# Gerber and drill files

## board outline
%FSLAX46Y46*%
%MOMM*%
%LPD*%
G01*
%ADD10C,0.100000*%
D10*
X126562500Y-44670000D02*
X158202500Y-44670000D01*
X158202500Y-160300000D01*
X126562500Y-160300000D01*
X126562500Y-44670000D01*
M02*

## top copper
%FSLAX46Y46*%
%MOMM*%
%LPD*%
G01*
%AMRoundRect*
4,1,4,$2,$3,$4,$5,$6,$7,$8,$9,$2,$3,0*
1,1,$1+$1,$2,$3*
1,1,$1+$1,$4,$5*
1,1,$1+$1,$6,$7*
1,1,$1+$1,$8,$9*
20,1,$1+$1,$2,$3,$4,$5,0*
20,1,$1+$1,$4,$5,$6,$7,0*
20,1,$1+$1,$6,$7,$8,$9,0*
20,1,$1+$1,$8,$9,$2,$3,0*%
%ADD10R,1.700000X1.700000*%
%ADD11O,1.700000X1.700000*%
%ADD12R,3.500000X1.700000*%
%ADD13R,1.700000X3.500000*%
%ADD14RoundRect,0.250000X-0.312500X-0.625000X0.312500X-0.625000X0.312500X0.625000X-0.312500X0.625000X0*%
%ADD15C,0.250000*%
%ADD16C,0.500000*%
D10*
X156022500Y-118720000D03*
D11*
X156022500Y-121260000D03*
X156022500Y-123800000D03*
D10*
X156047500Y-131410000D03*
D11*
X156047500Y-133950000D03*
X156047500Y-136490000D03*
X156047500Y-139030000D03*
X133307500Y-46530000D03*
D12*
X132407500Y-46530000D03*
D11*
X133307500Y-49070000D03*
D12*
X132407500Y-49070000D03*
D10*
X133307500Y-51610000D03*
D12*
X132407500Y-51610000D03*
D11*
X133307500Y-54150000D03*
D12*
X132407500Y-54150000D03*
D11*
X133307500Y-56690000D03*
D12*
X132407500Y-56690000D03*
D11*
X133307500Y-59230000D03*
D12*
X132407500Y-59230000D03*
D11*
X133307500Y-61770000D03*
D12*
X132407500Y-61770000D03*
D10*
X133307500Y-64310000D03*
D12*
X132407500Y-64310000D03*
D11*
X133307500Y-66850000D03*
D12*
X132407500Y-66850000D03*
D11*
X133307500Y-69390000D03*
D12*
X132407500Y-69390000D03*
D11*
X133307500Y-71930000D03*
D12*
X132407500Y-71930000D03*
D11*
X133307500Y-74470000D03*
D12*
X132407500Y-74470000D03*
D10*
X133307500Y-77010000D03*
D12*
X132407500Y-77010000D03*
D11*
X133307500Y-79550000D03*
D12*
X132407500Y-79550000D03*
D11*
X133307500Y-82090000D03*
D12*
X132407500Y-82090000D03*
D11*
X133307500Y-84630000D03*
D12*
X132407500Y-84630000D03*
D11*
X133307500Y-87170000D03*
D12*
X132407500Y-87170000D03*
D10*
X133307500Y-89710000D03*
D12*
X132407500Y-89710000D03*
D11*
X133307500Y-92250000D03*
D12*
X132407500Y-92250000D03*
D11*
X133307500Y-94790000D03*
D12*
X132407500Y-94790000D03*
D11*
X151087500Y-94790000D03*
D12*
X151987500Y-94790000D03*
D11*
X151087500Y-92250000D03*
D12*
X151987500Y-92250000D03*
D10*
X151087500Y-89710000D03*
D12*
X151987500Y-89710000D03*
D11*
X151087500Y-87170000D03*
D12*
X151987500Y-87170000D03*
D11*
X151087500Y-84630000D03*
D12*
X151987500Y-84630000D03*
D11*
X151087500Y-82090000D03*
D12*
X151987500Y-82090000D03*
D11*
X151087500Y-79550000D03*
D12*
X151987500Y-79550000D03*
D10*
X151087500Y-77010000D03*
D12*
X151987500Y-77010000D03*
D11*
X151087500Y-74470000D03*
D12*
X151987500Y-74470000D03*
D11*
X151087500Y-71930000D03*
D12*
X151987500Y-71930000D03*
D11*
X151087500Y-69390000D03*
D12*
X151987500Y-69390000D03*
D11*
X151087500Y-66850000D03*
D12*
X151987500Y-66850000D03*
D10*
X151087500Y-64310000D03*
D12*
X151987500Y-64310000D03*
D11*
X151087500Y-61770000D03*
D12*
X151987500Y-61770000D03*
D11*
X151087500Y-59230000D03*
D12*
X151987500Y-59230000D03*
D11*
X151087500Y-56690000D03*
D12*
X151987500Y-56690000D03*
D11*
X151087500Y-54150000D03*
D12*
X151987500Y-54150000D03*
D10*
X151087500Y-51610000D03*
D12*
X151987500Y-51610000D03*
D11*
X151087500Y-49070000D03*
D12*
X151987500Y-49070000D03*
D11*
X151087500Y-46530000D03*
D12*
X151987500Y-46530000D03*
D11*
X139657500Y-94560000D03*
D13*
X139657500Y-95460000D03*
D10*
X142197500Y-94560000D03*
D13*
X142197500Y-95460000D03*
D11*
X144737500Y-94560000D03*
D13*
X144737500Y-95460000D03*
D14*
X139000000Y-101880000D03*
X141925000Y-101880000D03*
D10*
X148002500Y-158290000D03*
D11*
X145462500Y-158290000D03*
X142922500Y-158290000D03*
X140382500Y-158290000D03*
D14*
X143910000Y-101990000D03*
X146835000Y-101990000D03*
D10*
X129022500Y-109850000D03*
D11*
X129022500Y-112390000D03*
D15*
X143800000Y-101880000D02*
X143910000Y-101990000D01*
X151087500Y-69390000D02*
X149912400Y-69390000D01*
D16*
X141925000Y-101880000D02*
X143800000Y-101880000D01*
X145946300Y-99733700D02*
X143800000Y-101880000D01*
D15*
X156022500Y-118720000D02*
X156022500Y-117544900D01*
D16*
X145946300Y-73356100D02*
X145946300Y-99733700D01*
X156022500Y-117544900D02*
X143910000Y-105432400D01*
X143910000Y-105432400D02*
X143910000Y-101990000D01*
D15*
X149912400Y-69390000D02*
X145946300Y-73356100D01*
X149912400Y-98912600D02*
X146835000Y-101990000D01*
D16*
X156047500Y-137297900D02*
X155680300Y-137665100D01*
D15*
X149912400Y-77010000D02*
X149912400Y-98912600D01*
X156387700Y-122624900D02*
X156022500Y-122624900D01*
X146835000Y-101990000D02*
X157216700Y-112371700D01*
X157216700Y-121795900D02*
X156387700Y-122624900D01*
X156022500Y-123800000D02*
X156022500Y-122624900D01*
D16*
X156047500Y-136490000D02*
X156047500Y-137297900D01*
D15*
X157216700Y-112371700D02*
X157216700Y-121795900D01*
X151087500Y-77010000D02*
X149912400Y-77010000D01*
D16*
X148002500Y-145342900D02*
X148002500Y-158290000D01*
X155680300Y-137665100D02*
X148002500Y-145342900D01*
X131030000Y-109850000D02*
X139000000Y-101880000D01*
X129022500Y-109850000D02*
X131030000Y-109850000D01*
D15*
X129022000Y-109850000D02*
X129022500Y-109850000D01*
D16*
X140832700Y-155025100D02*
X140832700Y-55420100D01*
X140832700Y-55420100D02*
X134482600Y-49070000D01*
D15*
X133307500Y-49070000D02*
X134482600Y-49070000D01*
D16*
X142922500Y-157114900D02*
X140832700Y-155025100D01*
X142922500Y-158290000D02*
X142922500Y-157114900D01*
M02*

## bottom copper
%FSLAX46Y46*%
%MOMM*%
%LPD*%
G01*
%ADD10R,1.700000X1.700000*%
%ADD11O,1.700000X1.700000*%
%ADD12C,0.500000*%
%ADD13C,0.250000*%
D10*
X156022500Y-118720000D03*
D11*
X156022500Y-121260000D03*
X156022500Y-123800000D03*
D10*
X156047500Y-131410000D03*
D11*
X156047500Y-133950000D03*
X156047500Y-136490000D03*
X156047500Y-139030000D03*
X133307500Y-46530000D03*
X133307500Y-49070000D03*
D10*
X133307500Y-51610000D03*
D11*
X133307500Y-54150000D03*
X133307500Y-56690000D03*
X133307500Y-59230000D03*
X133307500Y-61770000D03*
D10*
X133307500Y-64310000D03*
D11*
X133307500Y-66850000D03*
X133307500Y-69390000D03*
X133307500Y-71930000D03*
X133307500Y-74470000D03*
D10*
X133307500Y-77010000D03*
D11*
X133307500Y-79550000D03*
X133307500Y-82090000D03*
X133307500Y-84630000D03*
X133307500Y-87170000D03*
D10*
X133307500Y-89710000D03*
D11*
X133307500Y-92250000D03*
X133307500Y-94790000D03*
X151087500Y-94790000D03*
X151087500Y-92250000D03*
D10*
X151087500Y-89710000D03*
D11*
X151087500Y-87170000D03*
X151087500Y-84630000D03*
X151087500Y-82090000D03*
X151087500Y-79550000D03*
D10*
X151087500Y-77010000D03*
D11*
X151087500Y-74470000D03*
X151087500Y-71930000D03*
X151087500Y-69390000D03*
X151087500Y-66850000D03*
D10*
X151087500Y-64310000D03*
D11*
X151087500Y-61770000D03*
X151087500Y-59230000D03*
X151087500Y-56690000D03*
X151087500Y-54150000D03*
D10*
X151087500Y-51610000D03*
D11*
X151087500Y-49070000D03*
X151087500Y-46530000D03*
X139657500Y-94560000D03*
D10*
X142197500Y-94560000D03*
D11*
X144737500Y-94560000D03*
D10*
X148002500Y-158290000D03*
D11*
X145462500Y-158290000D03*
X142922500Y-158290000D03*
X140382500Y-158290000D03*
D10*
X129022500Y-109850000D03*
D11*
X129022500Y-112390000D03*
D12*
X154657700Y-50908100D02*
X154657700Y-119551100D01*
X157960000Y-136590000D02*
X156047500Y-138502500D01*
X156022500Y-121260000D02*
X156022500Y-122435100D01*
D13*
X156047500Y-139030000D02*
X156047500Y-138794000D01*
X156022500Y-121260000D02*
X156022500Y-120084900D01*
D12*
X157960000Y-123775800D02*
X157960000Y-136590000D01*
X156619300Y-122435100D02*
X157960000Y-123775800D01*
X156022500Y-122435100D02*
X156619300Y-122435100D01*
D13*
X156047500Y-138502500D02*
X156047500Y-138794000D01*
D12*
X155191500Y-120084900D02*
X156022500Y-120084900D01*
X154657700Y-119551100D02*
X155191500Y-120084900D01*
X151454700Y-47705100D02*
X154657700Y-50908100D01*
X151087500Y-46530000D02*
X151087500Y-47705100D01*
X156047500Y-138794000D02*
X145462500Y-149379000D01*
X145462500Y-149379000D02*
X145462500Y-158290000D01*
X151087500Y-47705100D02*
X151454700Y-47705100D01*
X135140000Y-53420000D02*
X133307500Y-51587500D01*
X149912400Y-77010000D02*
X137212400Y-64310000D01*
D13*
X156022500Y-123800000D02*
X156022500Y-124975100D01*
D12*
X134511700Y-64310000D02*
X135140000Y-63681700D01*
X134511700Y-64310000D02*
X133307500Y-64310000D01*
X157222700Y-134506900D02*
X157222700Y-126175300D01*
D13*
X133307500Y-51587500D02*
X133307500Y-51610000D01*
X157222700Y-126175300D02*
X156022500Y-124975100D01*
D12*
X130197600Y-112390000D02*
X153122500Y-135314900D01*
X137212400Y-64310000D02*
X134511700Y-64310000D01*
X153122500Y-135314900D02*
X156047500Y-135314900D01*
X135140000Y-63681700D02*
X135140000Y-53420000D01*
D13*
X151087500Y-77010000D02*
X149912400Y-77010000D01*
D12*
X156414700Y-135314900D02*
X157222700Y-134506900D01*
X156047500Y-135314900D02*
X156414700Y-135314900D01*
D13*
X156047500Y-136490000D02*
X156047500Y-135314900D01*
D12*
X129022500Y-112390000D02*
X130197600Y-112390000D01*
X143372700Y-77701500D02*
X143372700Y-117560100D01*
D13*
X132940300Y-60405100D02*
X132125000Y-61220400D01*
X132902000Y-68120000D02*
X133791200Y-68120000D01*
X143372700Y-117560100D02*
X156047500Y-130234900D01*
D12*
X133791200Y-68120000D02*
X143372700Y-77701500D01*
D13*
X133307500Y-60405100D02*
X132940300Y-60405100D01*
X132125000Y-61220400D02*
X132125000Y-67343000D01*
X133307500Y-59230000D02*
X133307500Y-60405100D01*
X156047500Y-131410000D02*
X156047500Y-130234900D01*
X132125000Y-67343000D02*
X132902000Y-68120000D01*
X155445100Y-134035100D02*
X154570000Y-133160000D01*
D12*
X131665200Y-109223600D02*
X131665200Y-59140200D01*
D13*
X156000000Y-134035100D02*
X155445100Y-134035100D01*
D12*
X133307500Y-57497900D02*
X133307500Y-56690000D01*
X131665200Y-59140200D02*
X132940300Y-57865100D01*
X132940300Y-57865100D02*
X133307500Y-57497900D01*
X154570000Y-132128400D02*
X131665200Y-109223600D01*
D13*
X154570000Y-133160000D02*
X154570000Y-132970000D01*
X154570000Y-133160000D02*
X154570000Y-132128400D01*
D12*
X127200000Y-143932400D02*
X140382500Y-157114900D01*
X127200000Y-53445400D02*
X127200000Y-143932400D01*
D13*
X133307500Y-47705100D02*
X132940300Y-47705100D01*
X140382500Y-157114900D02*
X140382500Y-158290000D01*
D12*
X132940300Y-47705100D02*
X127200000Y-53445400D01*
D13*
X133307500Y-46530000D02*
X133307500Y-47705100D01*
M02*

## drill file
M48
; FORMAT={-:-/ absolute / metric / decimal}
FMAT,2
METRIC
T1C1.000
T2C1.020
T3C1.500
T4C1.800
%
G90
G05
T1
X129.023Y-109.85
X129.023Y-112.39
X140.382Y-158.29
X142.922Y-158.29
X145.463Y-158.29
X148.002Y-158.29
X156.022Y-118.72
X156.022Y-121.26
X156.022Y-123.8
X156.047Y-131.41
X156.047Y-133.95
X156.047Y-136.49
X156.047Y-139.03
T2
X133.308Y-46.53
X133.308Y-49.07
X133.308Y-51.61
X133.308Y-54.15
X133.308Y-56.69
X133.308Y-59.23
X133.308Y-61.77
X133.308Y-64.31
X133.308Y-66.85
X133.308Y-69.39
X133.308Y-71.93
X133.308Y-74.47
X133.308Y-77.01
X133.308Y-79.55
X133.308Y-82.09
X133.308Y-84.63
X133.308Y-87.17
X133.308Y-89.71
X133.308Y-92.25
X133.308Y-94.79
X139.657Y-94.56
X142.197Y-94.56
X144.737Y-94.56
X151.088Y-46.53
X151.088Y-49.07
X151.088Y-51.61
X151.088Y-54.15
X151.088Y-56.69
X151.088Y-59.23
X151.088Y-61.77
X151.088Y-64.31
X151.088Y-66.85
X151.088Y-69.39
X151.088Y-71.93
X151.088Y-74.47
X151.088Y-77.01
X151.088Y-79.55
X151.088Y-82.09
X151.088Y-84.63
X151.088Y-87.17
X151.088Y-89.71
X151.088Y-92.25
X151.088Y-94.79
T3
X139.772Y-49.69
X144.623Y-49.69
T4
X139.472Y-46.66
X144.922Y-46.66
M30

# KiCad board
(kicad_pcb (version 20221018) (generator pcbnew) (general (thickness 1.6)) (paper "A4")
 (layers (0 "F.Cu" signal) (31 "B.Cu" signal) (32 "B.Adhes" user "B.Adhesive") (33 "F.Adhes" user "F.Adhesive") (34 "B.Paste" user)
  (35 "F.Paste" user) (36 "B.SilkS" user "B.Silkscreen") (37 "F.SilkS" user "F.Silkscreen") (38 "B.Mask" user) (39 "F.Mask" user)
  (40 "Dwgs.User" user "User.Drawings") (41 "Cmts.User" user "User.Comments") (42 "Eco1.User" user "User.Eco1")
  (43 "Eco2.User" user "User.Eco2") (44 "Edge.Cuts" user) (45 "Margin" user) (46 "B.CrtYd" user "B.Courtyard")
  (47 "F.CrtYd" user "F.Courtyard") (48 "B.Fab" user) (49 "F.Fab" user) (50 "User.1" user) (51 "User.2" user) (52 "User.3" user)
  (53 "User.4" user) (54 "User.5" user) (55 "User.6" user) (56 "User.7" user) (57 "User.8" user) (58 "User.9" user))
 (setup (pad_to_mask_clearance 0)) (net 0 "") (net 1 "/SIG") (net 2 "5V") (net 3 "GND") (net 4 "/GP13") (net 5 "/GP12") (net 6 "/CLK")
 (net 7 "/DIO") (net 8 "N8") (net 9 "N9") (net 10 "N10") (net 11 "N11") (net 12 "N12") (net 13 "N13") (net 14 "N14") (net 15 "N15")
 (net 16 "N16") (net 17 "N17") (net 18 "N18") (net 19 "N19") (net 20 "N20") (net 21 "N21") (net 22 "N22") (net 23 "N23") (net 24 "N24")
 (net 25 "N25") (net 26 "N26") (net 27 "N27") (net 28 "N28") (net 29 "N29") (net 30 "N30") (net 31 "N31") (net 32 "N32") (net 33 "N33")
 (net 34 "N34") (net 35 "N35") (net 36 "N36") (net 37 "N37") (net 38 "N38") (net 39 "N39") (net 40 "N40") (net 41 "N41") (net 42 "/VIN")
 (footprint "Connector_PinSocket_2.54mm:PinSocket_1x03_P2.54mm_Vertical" (layer "F.Cu") (at 156.0225 118.72)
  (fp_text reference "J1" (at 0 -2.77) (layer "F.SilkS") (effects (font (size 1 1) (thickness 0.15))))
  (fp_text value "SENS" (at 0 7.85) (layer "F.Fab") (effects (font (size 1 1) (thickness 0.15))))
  (pad "1" thru_hole rect (at 0 0) (size 1.7 1.7) (drill 1) (layers "*.Cu" "*.Mask") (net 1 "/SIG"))
  (pad "2" thru_hole oval (at 0 2.54) (size 1.7 1.7) (drill 1) (layers "*.Cu" "*.Mask") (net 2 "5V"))
  (pad "3" thru_hole oval (at 0 5.08) (size 1.7 1.7) (drill 1) (layers "*.Cu" "*.Mask") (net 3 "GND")))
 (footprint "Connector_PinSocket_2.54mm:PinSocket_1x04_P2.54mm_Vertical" (layer "F.Cu") (at 156.0475 131.41)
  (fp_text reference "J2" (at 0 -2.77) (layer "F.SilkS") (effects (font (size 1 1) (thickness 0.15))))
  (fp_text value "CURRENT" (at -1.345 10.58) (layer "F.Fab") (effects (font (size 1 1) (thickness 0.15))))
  (pad "1" thru_hole rect (at 0 0) (size 1.7 1.7) (drill 1) (layers "*.Cu" "*.Mask") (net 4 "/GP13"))
  (pad "2" thru_hole oval (at 0 2.54) (size 1.7 1.7) (drill 1) (layers "*.Cu" "*.Mask") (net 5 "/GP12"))
  (pad "3" thru_hole oval (at 0 5.08) (size 1.7 1.7) (drill 1) (layers "*.Cu" "*.Mask") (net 3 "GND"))
  (pad "4" thru_hole oval (at 0 7.62) (size 1.7 1.7) (drill 1) (layers "*.Cu" "*.Mask") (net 2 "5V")))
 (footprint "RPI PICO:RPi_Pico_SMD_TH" (layer "F.Cu") (at 142.1975 70.66)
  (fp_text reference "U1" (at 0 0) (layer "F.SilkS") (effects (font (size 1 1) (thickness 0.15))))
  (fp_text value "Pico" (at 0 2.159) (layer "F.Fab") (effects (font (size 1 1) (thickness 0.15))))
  (pad "" np_thru_hole oval (at -2.725 -24) (size 1.8 1.8) (drill 1.8) (layers "*.Cu" "*.Mask"))
  (pad "" np_thru_hole oval (at -2.425 -20.97) (size 1.5 1.5) (drill 1.5) (layers "*.Cu" "*.Mask"))
  (pad "" np_thru_hole oval (at 2.425 -20.97) (size 1.5 1.5) (drill 1.5) (layers "*.Cu" "*.Mask"))
  (pad "" np_thru_hole oval (at 2.725 -24) (size 1.8 1.8) (drill 1.8) (layers "*.Cu" "*.Mask"))
  (pad "1" thru_hole oval (at -8.89 -24.13) (size 1.7 1.7) (drill 1.02) (layers "*.Cu" "*.Mask") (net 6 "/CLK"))
  (pad "1" smd rect (at -8.89 -24.13) (size 3.5 1.7) (drill (offset -0.9 0)) (layers "F.Cu" "F.Mask") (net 6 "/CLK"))
  (pad "2" thru_hole oval (at -8.89 -21.59) (size 1.7 1.7) (drill 1.02) (layers "*.Cu" "*.Mask") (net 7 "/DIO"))
  (pad "2" smd rect (at -8.89 -21.59) (size 3.5 1.7) (drill (offset -0.9 0)) (layers "F.Cu" "F.Mask") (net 7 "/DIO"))
  (pad "3" thru_hole rect (at -8.89 -19.05) (size 1.7 1.7) (drill 1.02) (layers "*.Cu" "*.Mask") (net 3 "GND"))
  (pad "3" smd rect (at -8.89 -19.05) (size 3.5 1.7) (drill (offset -0.9 0)) (layers "F.Cu" "F.Mask") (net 3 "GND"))
  (pad "4" thru_hole oval (at -8.89 -16.51) (size 1.7 1.7) (drill 1.02) (layers "*.Cu" "*.Mask") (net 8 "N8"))
  (pad "4" smd rect (at -8.89 -16.51) (size 3.5 1.7) (drill (offset -0.9 0)) (layers "F.Cu" "F.Mask") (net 8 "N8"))
  (pad "5" thru_hole oval (at -8.89 -13.97) (size 1.7 1.7) (drill 1.02) (layers "*.Cu" "*.Mask") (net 5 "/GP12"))
  (pad "5" smd rect (at -8.89 -13.97) (size 3.5 1.7) (drill (offset -0.9 0)) (layers "F.Cu" "F.Mask") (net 5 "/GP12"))
  (pad "6" thru_hole oval (at -8.89 -11.43) (size 1.7 1.7) (drill 1.02) (layers "*.Cu" "*.Mask") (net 4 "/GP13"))
  (pad "6" smd rect (at -8.89 -11.43) (size 3.5 1.7) (drill (offset -0.9 0)) (layers "F.Cu" "F.Mask") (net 4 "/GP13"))
  (pad "7" thru_hole oval (at -8.89 -8.89) (size 1.7 1.7) (drill 1.02) (layers "*.Cu" "*.Mask") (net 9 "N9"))
  (pad "7" smd rect (at -8.89 -8.89) (size 3.5 1.7) (drill (offset -0.9 0)) (layers "F.Cu" "F.Mask") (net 9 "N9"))
  (pad "8" thru_hole rect (at -8.89 -6.35) (size 1.7 1.7) (drill 1.02) (layers "*.Cu" "*.Mask") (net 3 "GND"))
  (pad "8" smd rect (at -8.89 -6.35) (size 3.5 1.7) (drill (offset -0.9 0)) (layers "F.Cu" "F.Mask") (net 3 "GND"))
  (pad "9" thru_hole oval (at -8.89 -3.81) (size 1.7 1.7) (drill 1.02) (layers "*.Cu" "*.Mask") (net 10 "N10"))
  (pad "9" smd rect (at -8.89 -3.81) (size 3.5 1.7) (drill (offset -0.9 0)) (layers "F.Cu" "F.Mask") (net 10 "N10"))
  (pad "10" thru_hole oval (at -8.89 -1.27) (size 1.7 1.7) (drill 1.02) (layers "*.Cu" "*.Mask") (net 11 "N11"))
  (pad "10" smd rect (at -8.89 -1.27) (size 3.5 1.7) (drill (offset -0.9 0)) (layers "F.Cu" "F.Mask") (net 11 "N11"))
  (pad "11" thru_hole oval (at -8.89 1.27) (size 1.7 1.7) (drill 1.02) (layers "*.Cu" "*.Mask") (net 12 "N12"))
  (pad "11" smd rect (at -8.89 1.27) (size 3.5 1.7) (drill (offset -0.9 0)) (layers "F.Cu" "F.Mask") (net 12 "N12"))
  (pad "12" thru_hole oval (at -8.89 3.81) (size 1.7 1.7) (drill 1.02) (layers "*.Cu" "*.Mask") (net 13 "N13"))
  (pad "12" smd rect (at -8.89 3.81) (size 3.5 1.7) (drill (offset -0.9 0)) (layers "F.Cu" "F.Mask") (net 13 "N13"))
  (pad "13" thru_hole rect (at -8.89 6.35) (size 1.7 1.7) (drill 1.02) (layers "*.Cu" "*.Mask") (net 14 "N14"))
  (pad "13" smd rect (at -8.89 6.35) (size 3.5 1.7) (drill (offset -0.9 0)) (layers "F.Cu" "F.Mask") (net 14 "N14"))
  (pad "14" thru_hole oval (at -8.89 8.89) (size 1.7 1.7) (drill 1.02) (layers "*.Cu" "*.Mask") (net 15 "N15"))
  (pad "14" smd rect (at -8.89 8.89) (size 3.5 1.7) (drill (offset -0.9 0)) (layers "F.Cu" "F.Mask") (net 15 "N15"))
  (pad "15" thru_hole oval (at -8.89 11.43) (size 1.7 1.7) (drill 1.02) (layers "*.Cu" "*.Mask") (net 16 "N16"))
  (pad "15" smd rect (at -8.89 11.43) (size 3.5 1.7) (drill (offset -0.9 0)) (layers "F.Cu" "F.Mask") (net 16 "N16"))
  (pad "16" thru_hole oval (at -8.89 13.97) (size 1.7 1.7) (drill 1.02) (layers "*.Cu" "*.Mask") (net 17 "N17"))
  (pad "16" smd rect (at -8.89 13.97) (size 3.5 1.7) (drill (offset -0.9 0)) (layers "F.Cu" "F.Mask") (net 17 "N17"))
  (pad "17" thru_hole oval (at -8.89 16.51) (size 1.7 1.7) (drill 1.02) (layers "*.Cu" "*.Mask") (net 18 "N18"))
  (pad "17" smd rect (at -8.89 16.51) (size 3.5 1.7) (drill (offset -0.9 0)) (layers "F.Cu" "F.Mask") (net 18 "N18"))
  (pad "18" thru_hole rect (at -8.89 19.05) (size 1.7 1.7) (drill 1.02) (layers "*.Cu" "*.Mask") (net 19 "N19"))
  (pad "18" smd rect (at -8.89 19.05) (size 3.5 1.7) (drill (offset -0.9 0)) (layers "F.Cu" "F.Mask") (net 19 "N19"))
  (pad "19" thru_hole oval (at -8.89 21.59) (size 1.7 1.7) (drill 1.02) (layers "*.Cu" "*.Mask") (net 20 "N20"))
  (pad "19" smd rect (at -8.89 21.59) (size 3.5 1.7) (drill (offset -0.9 0)) (layers "F.Cu" "F.Mask") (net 20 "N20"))
  (pad "20" thru_hole oval (at -8.89 24.13) (size 1.7 1.7) (drill 1.02) (layers "*.Cu" "*.Mask") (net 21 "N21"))
  (pad "20" smd rect (at -8.89 24.13) (size 3.5 1.7) (drill (offset -0.9 0)) (layers "F.Cu" "F.Mask") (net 21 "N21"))
  (pad "21" thru_hole oval (at 8.89 24.13) (size 1.7 1.7) (drill 1.02) (layers "*.Cu" "*.Mask") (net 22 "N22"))
  (pad "21" smd rect (at 8.89 24.13) (size 3.5 1.7) (drill (offset 0.9 0)) (layers "F.Cu" "F.Mask") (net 22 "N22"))
  (pad "22" thru_hole oval (at 8.89 21.59) (size 1.7 1.7) (drill 1.02) (layers "*.Cu" "*.Mask") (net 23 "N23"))
  (pad "22" smd rect (at 8.89 21.59) (size 3.5 1.7) (drill (offset 0.9 0)) (layers "F.Cu" "F.Mask") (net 23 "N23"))
  (pad "23" thru_hole rect (at 8.89 19.05) (size 1.7 1.7) (drill 1.02) (layers "*.Cu" "*.Mask") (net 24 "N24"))
  (pad "23" smd rect (at 8.89 19.05) (size 3.5 1.7) (drill (offset 0.9 0)) (layers "F.Cu" "F.Mask") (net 24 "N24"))
  (pad "24" thru_hole oval (at 8.89 16.51) (size 1.7 1.7) (drill 1.02) (layers "*.Cu" "*.Mask") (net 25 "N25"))
  (pad "24" smd rect (at 8.89 16.51) (size 3.5 1.7) (drill (offset 0.9 0)) (layers "F.Cu" "F.Mask") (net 25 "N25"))
  (pad "25" thru_hole oval (at 8.89 13.97) (size 1.7 1.7) (drill 1.02) (layers "*.Cu" "*.Mask") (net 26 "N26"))
  (pad "25" smd rect (at 8.89 13.97) (size 3.5 1.7) (drill (offset 0.9 0)) (layers "F.Cu" "F.Mask") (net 26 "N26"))
  (pad "26" thru_hole oval (at 8.89 11.43) (size 1.7 1.7) (drill 1.02) (layers "*.Cu" "*.Mask") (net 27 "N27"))
  (pad "26" smd rect (at 8.89 11.43) (size 3.5 1.7) (drill (offset 0.9 0)) (layers "F.Cu" "F.Mask") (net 27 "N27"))
  (pad "27" thru_hole oval (at 8.89 8.89) (size 1.7 1.7) (drill 1.02) (layers "*.Cu" "*.Mask") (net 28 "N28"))
  (pad "27" smd rect (at 8.89 8.89) (size 3.5 1.7) (drill (offset 0.9 0)) (layers "F.Cu" "F.Mask") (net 28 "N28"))
  (pad "28" thru_hole rect (at 8.89 6.35) (size 1.7 1.7) (drill 1.02) (layers "*.Cu" "*.Mask") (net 3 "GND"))
  (pad "28" smd rect (at 8.89 6.35) (size 3.5 1.7) (drill (offset 0.9 0)) (layers "F.Cu" "F.Mask") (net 3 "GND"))
  (pad "29" thru_hole oval (at 8.89 3.81) (size 1.7 1.7) (drill 1.02) (layers "*.Cu" "*.Mask") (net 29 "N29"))
  (pad "29" smd rect (at 8.89 3.81) (size 3.5 1.7) (drill (offset 0.9 0)) (layers "F.Cu" "F.Mask") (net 29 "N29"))
  (pad "30" thru_hole oval (at 8.89 1.27) (size 1.7 1.7) (drill 1.02) (layers "*.Cu" "*.Mask") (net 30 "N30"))
  (pad "30" smd rect (at 8.89 1.27) (size 3.5 1.7) (drill (offset 0.9 0)) (layers "F.Cu" "F.Mask") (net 30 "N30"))
  (pad "31" thru_hole oval (at 8.89 -1.27) (size 1.7 1.7) (drill 1.02) (layers "*.Cu" "*.Mask") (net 1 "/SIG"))
  (pad "31" smd rect (at 8.89 -1.27) (size 3.5 1.7) (drill (offset 0.9 0)) (layers "F.Cu" "F.Mask") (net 1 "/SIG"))
  (pad "32" thru_hole oval (at 8.89 -3.81) (size 1.7 1.7) (drill 1.02) (layers "*.Cu" "*.Mask") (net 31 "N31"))
  (pad "32" smd rect (at 8.89 -3.81) (size 3.5 1.7) (drill (offset 0.9 0)) (layers "F.Cu" "F.Mask") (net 31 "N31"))
  (pad "33" thru_hole rect (at 8.89 -6.35) (size 1.7 1.7) (drill 1.02) (layers "*.Cu" "*.Mask") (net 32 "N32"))
  (pad "33" smd rect (at 8.89 -6.35) (size 3.5 1.7) (drill (offset 0.9 0)) (layers "F.Cu" "F.Mask") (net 32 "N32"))
  (pad "34" thru_hole oval (at 8.89 -8.89) (size 1.7 1.7) (drill 1.02) (layers "*.Cu" "*.Mask") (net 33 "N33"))
  (pad "34" smd rect (at 8.89 -8.89) (size 3.5 1.7) (drill (offset 0.9 0)) (layers "F.Cu" "F.Mask") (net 33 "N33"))
  (pad "35" thru_hole oval (at 8.89 -11.43) (size 1.7 1.7) (drill 1.02) (layers "*.Cu" "*.Mask") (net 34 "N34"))
  (pad "35" smd rect (at 8.89 -11.43) (size 3.5 1.7) (drill (offset 0.9 0)) (layers "F.Cu" "F.Mask") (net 34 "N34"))
  (pad "36" thru_hole oval (at 8.89 -13.97) (size 1.7 1.7) (drill 1.02) (layers "*.Cu" "*.Mask") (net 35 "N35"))
  (pad "36" smd rect (at 8.89 -13.97) (size 3.5 1.7) (drill (offset 0.9 0)) (layers "F.Cu" "F.Mask") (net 35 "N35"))
  (pad "37" thru_hole oval (at 8.89 -16.51) (size 1.7 1.7) (drill 1.02) (layers "*.Cu" "*.Mask") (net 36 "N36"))
  (pad "37" smd rect (at 8.89 -16.51) (size 3.5 1.7) (drill (offset 0.9 0)) (layers "F.Cu" "F.Mask") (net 36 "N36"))
  (pad "38" thru_hole rect (at 8.89 -19.05) (size 1.7 1.7) (drill 1.02) (layers "*.Cu" "*.Mask") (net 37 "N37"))
  (pad "38" smd rect (at 8.89 -19.05) (size 3.5 1.7) (drill (offset 0.9 0)) (layers "F.Cu" "F.Mask") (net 37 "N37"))
  (pad "39" thru_hole oval (at 8.89 -21.59) (size 1.7 1.7) (drill 1.02) (layers "*.Cu" "*.Mask") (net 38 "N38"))
  (pad "39" smd rect (at 8.89 -21.59) (size 3.5 1.7) (drill (offset 0.9 0)) (layers "F.Cu" "F.Mask") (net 38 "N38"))
  (pad "40" thru_hole oval (at 8.89 -24.13) (size 1.7 1.7) (drill 1.02) (layers "*.Cu" "*.Mask") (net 2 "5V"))
  (pad "40" smd rect (at 8.89 -24.13) (size 3.5 1.7) (drill (offset 0.9 0)) (layers "F.Cu" "F.Mask") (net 2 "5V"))
  (pad "41" thru_hole oval (at -2.54 23.9) (size 1.7 1.7) (drill 1.02) (layers "*.Cu" "*.Mask") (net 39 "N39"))
  (pad "41" smd rect (at -2.54 23.9 90) (size 3.5 1.7) (drill (offset -0.9 0)) (layers "F.Cu" "F.Mask") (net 39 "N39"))
  (pad "42" thru_hole rect (at 0 23.9) (size 1.7 1.7) (drill 1.02) (layers "*.Cu" "*.Mask") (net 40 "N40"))
  (pad "42" smd rect (at 0 23.9 90) (size 3.5 1.7) (drill (offset -0.9 0)) (layers "F.Cu" "F.Mask") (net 40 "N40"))
  (pad "43" thru_hole oval (at 2.54 23.9) (size 1.7 1.7) (drill 1.02) (layers "*.Cu" "*.Mask") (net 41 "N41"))
  (pad "43" smd rect (at 2.54 23.9 90) (size 3.5 1.7) (drill (offset -0.9 0)) (layers "F.Cu" "F.Mask") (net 41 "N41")))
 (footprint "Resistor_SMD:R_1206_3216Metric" (layer "F.Cu") (at 140.4625 101.88)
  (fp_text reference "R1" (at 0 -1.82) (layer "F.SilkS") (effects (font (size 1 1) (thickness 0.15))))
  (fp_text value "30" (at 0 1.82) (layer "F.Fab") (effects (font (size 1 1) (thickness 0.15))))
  (pad "1" smd roundrect (at -1.4625 0) (size 1.125 1.75) (layers "F.Cu" "F.Paste" "F.Mask") (roundrect_rratio 0.222222) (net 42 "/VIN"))
  (pad "2" smd roundrect (at 1.4625 0) (size 1.125 1.75) (layers "F.Cu" "F.Paste" "F.Mask") (roundrect_rratio 0.222222) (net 1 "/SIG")))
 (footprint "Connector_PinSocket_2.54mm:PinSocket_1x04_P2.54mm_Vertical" (layer "F.Cu") (at 148.0025 158.29 -90)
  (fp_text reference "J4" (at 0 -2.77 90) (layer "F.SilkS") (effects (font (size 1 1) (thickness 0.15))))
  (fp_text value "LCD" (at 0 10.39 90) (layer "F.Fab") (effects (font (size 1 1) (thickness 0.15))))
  (pad "1" thru_hole rect (at 0 0 270) (size 1.7 1.7) (drill 1) (layers "*.Cu" "*.Mask") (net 3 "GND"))
  (pad "2" thru_hole oval (at 0 2.54 270) (size 1.7 1.7) (drill 1) (layers "*.Cu" "*.Mask") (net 2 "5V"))
  (pad "3" thru_hole oval (at 0 5.08 270) (size 1.7 1.7) (drill 1) (layers "*.Cu" "*.Mask") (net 7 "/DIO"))
  (pad "4" thru_hole oval (at 0 7.62 270) (size 1.7 1.7) (drill 1) (layers "*.Cu" "*.Mask") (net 6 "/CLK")))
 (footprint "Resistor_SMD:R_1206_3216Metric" (layer "F.Cu") (at 145.3725 101.99)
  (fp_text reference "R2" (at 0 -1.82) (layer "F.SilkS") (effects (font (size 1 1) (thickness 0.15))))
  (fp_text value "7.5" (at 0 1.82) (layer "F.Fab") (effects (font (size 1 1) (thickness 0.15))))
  (pad "1" smd roundrect (at -1.4625 0) (size 1.125 1.75) (layers "F.Cu" "F.Paste" "F.Mask") (roundrect_rratio 0.222222) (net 1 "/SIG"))
  (pad "2" smd roundrect (at 1.4625 0) (size 1.125 1.75) (layers "F.Cu" "F.Paste" "F.Mask") (roundrect_rratio 0.222222) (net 3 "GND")))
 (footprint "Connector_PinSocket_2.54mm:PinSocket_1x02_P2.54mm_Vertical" (layer "F.Cu") (at 129.0225 109.85)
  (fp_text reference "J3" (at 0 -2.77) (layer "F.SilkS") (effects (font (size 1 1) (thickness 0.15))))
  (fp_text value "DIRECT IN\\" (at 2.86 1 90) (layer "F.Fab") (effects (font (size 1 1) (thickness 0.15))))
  (pad "1" thru_hole rect (at 0 0) (size 1.7 1.7) (drill 1) (layers "*.Cu" "*.Mask") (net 42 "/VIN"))
  (pad "2" thru_hole oval (at 0 2.54) (size 1.7 1.7) (drill 1) (layers "*.Cu" "*.Mask") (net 3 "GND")))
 (gr_rect (start 126.5625 44.67) (end 158.2025 160.3) (stroke (width 0.1) (type default)) (fill none) (layer "Edge.Cuts"))
 (segment (start 143.8 101.88) (end 143.91 101.99) (width 0.25) (layer "F.Cu") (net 1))
 (segment (start 151.0875 69.39) (end 149.9124 69.39) (width 0.25) (layer "F.Cu") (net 1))
 (segment (start 141.925 101.88) (end 143.8 101.88) (width 0.5) (layer "F.Cu") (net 1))
 (segment (start 145.9463 99.7337) (end 143.8 101.88) (width 0.5) (layer "F.Cu") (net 1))
 (segment (start 156.0225 118.72) (end 156.0225 117.5449) (width 0.25) (layer "F.Cu") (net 1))
 (segment (start 145.9463 73.3561) (end 145.9463 99.7337) (width 0.5) (layer "F.Cu") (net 1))
 (segment (start 156.0225 117.5449) (end 143.91 105.4324) (width 0.5) (layer "F.Cu") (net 1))
 (segment (start 143.91 105.4324) (end 143.91 101.99) (width 0.5) (layer "F.Cu") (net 1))
 (segment (start 149.9124 69.39) (end 145.9463 73.3561) (width 0.25) (layer "F.Cu") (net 1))
 (segment (start 154.6577 50.9081) (end 154.6577 119.5511) (width 0.5) (layer "B.Cu") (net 2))
 (segment (start 157.96 136.59) (end 156.0475 138.5025) (width 0.5) (layer "B.Cu") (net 2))
 (segment (start 156.0225 121.26) (end 156.0225 122.4351) (width 0.5) (layer "B.Cu") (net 2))
 (segment (start 156.0475 139.03) (end 156.0475 138.794) (width 0.25) (layer "B.Cu") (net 2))
 (segment (start 156.0225 121.26) (end 156.0225 120.0849) (width 0.25) (layer "B.Cu") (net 2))
 (segment (start 157.96 123.7758) (end 157.96 136.59) (width 0.5) (layer "B.Cu") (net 2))
 (segment (start 156.6193 122.4351) (end 157.96 123.7758) (width 0.5) (layer "B.Cu") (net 2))
 (segment (start 156.0225 122.4351) (end 156.6193 122.4351) (width 0.5) (layer "B.Cu") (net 2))
 (segment (start 156.0475 138.5025) (end 156.0475 138.794) (width 0.25) (layer "B.Cu") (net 2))
 (segment (start 155.1915 120.0849) (end 156.0225 120.0849) (width 0.5) (layer "B.Cu") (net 2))
 (segment (start 154.6577 119.5511) (end 155.1915 120.0849) (width 0.5) (layer "B.Cu") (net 2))
 (segment (start 151.4547 47.7051) (end 154.6577 50.9081) (width 0.5) (layer "B.Cu") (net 2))
 (segment (start 151.0875 46.53) (end 151.0875 47.7051) (width 0.5) (layer "B.Cu") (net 2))
 (segment (start 156.0475 138.794) (end 145.4625 149.379) (width 0.5) (layer "B.Cu") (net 2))
 (segment (start 145.4625 149.379) (end 145.4625 158.29) (width 0.5) (layer "B.Cu") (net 2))
 (segment (start 151.0875 47.7051) (end 151.4547 47.7051) (width 0.5) (layer "B.Cu") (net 2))
 (segment (start 149.9124 98.9126) (end 146.835 101.99) (width 0.25) (layer "F.Cu") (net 3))
 (segment (start 156.0475 137.2979) (end 155.6803 137.6651) (width 0.5) (layer "F.Cu") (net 3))
 (segment (start 149.9124 77.01) (end 149.9124 98.9126) (width 0.25) (layer "F.Cu") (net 3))
 (segment (start 156.3877 122.6249) (end 156.0225 122.6249) (width 0.25) (layer "F.Cu") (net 3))
 (segment (start 146.835 101.99) (end 157.2167 112.3717) (width 0.25) (layer "F.Cu") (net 3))
 (segment (start 157.2167 121.7959) (end 156.3877 122.6249) (width 0.25) (layer "F.Cu") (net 3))
 (segment (start 156.0225 123.8) (end 156.0225 122.6249) (width 0.25) (layer "F.Cu") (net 3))
 (segment (start 156.0475 136.49) (end 156.0475 137.2979) (width 0.5) (layer "F.Cu") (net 3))
 (segment (start 157.2167 112.3717) (end 157.2167 121.7959) (width 0.25) (layer "F.Cu") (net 3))
 (segment (start 151.0875 77.01) (end 149.9124 77.01) (width 0.25) (layer "F.Cu") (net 3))
 (segment (start 148.0025 145.3429) (end 148.0025 158.29) (width 0.5) (layer "F.Cu") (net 3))
 (segment (start 155.6803 137.6651) (end 148.0025 145.3429) (width 0.5) (layer "F.Cu") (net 3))
 (segment (start 135.14 53.42) (end 133.3075 51.5875) (width 0.5) (layer "B.Cu") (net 3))
 (segment (start 149.9124 77.01) (end 137.2124 64.31) (width 0.5) (layer "B.Cu") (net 3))
 (segment (start 156.0225 123.8) (end 156.0225 124.9751) (width 0.25) (layer "B.Cu") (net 3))
 (segment (start 134.5117 64.31) (end 135.14 63.6817) (width 0.5) (layer "B.Cu") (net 3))
 (segment (start 134.5117 64.31) (end 133.3075 64.31) (width 0.5) (layer "B.Cu") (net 3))
 (segment (start 157.2227 134.5069) (end 157.2227 126.1753) (width 0.5) (layer "B.Cu") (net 3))
 (segment (start 133.3075 51.5875) (end 133.3075 51.61) (width 0.25) (layer "B.Cu") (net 3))
 (segment (start 157.2227 126.1753) (end 156.0225 124.9751) (width 0.25) (layer "B.Cu") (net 3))
 (segment (start 130.1976 112.39) (end 153.1225 135.3149) (width 0.5) (layer "B.Cu") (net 3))
 (segment (start 137.2124 64.31) (end 134.5117 64.31) (width 0.5) (layer "B.Cu") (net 3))
 (segment (start 153.1225 135.3149) (end 156.0475 135.3149) (width 0.5) (layer "B.Cu") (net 3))
 (segment (start 135.14 63.6817) (end 135.14 53.42) (width 0.5) (layer "B.Cu") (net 3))
 (segment (start 151.0875 77.01) (end 149.9124 77.01) (width 0.25) (layer "B.Cu") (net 3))
 (segment (start 156.4147 135.3149) (end 157.2227 134.5069) (width 0.5) (layer "B.Cu") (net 3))
 (segment (start 156.0475 135.3149) (end 156.4147 135.3149) (width 0.5) (layer "B.Cu") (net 3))
 (segment (start 156.0475 136.49) (end 156.0475 135.3149) (width 0.25) (layer "B.Cu") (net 3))
 (segment (start 129.0225 112.39) (end 130.1976 112.39) (width 0.5) (layer "B.Cu") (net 3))
 (segment (start 143.3727 77.7015) (end 143.3727 117.5601) (width 0.5) (layer "B.Cu") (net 4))
 (segment (start 132.9403 60.4051) (end 132.125 61.2204) (width 0.25) (layer "B.Cu") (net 4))
 (segment (start 132.902 68.12) (end 133.7912 68.12) (width 0.25) (layer "B.Cu") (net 4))
 (segment (start 143.3727 117.5601) (end 156.0475 130.2349) (width 0.25) (layer "B.Cu") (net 4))
 (segment (start 133.7912 68.12) (end 143.3727 77.7015) (width 0.5) (layer "B.Cu") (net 4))
 (segment (start 133.3075 60.4051) (end 132.9403 60.4051) (width 0.25) (layer "B.Cu") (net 4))
 (segment (start 132.125 61.2204) (end 132.125 67.343) (width 0.25) (layer "B.Cu") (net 4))
 (segment (start 133.3075 59.23) (end 133.3075 60.4051) (width 0.25) (layer "B.Cu") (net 4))
 (segment (start 156.0475 131.41) (end 156.0475 130.2349) (width 0.25) (layer "B.Cu") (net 4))
 (segment (start 132.125 67.343) (end 132.902 68.12) (width 0.25) (layer "B.Cu") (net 4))
 (segment (start 155.4451 134.0351) (end 154.57 133.16) (width 0.25) (layer "B.Cu") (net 5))
 (segment (start 131.6652 109.2236) (end 131.6652 59.1402) (width 0.5) (layer "B.Cu") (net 5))
 (segment (start 156 134.0351) (end 155.4451 134.0351) (width 0.25) (layer "B.Cu") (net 5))
 (segment (start 133.3075 57.4979) (end 133.3075 56.69) (width 0.5) (layer "B.Cu") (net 5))
 (segment (start 131.6652 59.1402) (end 132.9403 57.8651) (width 0.5) (layer "B.Cu") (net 5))
 (segment (start 132.9403 57.8651) (end 133.3075 57.4979) (width 0.5) (layer "B.Cu") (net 5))
 (segment (start 154.57 132.1284) (end 131.6652 109.2236) (width 0.5) (layer "B.Cu") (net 5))
 (segment (start 154.57 133.16) (end 154.57 132.97) (width 0.25) (layer "B.Cu") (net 5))
 (segment (start 154.57 133.16) (end 154.57 132.1284) (width 0.25) (layer "B.Cu") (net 5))
 (segment (start 131.03 109.85) (end 139 101.88) (width 0.5) (layer "F.Cu") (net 42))
 (segment (start 129.0225 109.85) (end 131.03 109.85) (width 0.5) (layer "F.Cu") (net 42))
 (segment (start 129.022 109.85) (end 129.0225 109.85) (width 0.25) (layer "F.Cu") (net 42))
 (segment (start 140.8327 155.0251) (end 140.8327 55.4201) (width 0.5) (layer "F.Cu") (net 7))
 (segment (start 140.8327 55.4201) (end 134.4826 49.07) (width 0.5) (layer "F.Cu") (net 7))
 (segment (start 133.3075 49.07) (end 134.4826 49.07) (width 0.25) (layer "F.Cu") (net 7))
 (segment (start 142.9225 157.1149) (end 140.8327 155.0251) (width 0.5) (layer "F.Cu") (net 7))
 (segment (start 142.9225 158.29) (end 142.9225 157.1149) (width 0.5) (layer "F.Cu") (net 7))
 (segment (start 127.2 143.9324) (end 140.3825 157.1149) (width 0.5) (layer "B.Cu") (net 6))
 (segment (start 127.2 53.4454) (end 127.2 143.9324) (width 0.5) (layer "B.Cu") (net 6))
 (segment (start 133.3075 47.7051) (end 132.9403 47.7051) (width 0.25) (layer "B.Cu") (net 6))
 (segment (start 140.3825 157.1149) (end 140.3825 158.29) (width 0.25) (layer "B.Cu") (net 6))
 (segment (start 132.9403 47.7051) (end 127.2 53.4454) (width 0.5) (layer "B.Cu") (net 6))
 (segment (start 133.3075 46.53) (end 133.3075 47.7051) (width 0.25) (layer "B.Cu") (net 6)))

